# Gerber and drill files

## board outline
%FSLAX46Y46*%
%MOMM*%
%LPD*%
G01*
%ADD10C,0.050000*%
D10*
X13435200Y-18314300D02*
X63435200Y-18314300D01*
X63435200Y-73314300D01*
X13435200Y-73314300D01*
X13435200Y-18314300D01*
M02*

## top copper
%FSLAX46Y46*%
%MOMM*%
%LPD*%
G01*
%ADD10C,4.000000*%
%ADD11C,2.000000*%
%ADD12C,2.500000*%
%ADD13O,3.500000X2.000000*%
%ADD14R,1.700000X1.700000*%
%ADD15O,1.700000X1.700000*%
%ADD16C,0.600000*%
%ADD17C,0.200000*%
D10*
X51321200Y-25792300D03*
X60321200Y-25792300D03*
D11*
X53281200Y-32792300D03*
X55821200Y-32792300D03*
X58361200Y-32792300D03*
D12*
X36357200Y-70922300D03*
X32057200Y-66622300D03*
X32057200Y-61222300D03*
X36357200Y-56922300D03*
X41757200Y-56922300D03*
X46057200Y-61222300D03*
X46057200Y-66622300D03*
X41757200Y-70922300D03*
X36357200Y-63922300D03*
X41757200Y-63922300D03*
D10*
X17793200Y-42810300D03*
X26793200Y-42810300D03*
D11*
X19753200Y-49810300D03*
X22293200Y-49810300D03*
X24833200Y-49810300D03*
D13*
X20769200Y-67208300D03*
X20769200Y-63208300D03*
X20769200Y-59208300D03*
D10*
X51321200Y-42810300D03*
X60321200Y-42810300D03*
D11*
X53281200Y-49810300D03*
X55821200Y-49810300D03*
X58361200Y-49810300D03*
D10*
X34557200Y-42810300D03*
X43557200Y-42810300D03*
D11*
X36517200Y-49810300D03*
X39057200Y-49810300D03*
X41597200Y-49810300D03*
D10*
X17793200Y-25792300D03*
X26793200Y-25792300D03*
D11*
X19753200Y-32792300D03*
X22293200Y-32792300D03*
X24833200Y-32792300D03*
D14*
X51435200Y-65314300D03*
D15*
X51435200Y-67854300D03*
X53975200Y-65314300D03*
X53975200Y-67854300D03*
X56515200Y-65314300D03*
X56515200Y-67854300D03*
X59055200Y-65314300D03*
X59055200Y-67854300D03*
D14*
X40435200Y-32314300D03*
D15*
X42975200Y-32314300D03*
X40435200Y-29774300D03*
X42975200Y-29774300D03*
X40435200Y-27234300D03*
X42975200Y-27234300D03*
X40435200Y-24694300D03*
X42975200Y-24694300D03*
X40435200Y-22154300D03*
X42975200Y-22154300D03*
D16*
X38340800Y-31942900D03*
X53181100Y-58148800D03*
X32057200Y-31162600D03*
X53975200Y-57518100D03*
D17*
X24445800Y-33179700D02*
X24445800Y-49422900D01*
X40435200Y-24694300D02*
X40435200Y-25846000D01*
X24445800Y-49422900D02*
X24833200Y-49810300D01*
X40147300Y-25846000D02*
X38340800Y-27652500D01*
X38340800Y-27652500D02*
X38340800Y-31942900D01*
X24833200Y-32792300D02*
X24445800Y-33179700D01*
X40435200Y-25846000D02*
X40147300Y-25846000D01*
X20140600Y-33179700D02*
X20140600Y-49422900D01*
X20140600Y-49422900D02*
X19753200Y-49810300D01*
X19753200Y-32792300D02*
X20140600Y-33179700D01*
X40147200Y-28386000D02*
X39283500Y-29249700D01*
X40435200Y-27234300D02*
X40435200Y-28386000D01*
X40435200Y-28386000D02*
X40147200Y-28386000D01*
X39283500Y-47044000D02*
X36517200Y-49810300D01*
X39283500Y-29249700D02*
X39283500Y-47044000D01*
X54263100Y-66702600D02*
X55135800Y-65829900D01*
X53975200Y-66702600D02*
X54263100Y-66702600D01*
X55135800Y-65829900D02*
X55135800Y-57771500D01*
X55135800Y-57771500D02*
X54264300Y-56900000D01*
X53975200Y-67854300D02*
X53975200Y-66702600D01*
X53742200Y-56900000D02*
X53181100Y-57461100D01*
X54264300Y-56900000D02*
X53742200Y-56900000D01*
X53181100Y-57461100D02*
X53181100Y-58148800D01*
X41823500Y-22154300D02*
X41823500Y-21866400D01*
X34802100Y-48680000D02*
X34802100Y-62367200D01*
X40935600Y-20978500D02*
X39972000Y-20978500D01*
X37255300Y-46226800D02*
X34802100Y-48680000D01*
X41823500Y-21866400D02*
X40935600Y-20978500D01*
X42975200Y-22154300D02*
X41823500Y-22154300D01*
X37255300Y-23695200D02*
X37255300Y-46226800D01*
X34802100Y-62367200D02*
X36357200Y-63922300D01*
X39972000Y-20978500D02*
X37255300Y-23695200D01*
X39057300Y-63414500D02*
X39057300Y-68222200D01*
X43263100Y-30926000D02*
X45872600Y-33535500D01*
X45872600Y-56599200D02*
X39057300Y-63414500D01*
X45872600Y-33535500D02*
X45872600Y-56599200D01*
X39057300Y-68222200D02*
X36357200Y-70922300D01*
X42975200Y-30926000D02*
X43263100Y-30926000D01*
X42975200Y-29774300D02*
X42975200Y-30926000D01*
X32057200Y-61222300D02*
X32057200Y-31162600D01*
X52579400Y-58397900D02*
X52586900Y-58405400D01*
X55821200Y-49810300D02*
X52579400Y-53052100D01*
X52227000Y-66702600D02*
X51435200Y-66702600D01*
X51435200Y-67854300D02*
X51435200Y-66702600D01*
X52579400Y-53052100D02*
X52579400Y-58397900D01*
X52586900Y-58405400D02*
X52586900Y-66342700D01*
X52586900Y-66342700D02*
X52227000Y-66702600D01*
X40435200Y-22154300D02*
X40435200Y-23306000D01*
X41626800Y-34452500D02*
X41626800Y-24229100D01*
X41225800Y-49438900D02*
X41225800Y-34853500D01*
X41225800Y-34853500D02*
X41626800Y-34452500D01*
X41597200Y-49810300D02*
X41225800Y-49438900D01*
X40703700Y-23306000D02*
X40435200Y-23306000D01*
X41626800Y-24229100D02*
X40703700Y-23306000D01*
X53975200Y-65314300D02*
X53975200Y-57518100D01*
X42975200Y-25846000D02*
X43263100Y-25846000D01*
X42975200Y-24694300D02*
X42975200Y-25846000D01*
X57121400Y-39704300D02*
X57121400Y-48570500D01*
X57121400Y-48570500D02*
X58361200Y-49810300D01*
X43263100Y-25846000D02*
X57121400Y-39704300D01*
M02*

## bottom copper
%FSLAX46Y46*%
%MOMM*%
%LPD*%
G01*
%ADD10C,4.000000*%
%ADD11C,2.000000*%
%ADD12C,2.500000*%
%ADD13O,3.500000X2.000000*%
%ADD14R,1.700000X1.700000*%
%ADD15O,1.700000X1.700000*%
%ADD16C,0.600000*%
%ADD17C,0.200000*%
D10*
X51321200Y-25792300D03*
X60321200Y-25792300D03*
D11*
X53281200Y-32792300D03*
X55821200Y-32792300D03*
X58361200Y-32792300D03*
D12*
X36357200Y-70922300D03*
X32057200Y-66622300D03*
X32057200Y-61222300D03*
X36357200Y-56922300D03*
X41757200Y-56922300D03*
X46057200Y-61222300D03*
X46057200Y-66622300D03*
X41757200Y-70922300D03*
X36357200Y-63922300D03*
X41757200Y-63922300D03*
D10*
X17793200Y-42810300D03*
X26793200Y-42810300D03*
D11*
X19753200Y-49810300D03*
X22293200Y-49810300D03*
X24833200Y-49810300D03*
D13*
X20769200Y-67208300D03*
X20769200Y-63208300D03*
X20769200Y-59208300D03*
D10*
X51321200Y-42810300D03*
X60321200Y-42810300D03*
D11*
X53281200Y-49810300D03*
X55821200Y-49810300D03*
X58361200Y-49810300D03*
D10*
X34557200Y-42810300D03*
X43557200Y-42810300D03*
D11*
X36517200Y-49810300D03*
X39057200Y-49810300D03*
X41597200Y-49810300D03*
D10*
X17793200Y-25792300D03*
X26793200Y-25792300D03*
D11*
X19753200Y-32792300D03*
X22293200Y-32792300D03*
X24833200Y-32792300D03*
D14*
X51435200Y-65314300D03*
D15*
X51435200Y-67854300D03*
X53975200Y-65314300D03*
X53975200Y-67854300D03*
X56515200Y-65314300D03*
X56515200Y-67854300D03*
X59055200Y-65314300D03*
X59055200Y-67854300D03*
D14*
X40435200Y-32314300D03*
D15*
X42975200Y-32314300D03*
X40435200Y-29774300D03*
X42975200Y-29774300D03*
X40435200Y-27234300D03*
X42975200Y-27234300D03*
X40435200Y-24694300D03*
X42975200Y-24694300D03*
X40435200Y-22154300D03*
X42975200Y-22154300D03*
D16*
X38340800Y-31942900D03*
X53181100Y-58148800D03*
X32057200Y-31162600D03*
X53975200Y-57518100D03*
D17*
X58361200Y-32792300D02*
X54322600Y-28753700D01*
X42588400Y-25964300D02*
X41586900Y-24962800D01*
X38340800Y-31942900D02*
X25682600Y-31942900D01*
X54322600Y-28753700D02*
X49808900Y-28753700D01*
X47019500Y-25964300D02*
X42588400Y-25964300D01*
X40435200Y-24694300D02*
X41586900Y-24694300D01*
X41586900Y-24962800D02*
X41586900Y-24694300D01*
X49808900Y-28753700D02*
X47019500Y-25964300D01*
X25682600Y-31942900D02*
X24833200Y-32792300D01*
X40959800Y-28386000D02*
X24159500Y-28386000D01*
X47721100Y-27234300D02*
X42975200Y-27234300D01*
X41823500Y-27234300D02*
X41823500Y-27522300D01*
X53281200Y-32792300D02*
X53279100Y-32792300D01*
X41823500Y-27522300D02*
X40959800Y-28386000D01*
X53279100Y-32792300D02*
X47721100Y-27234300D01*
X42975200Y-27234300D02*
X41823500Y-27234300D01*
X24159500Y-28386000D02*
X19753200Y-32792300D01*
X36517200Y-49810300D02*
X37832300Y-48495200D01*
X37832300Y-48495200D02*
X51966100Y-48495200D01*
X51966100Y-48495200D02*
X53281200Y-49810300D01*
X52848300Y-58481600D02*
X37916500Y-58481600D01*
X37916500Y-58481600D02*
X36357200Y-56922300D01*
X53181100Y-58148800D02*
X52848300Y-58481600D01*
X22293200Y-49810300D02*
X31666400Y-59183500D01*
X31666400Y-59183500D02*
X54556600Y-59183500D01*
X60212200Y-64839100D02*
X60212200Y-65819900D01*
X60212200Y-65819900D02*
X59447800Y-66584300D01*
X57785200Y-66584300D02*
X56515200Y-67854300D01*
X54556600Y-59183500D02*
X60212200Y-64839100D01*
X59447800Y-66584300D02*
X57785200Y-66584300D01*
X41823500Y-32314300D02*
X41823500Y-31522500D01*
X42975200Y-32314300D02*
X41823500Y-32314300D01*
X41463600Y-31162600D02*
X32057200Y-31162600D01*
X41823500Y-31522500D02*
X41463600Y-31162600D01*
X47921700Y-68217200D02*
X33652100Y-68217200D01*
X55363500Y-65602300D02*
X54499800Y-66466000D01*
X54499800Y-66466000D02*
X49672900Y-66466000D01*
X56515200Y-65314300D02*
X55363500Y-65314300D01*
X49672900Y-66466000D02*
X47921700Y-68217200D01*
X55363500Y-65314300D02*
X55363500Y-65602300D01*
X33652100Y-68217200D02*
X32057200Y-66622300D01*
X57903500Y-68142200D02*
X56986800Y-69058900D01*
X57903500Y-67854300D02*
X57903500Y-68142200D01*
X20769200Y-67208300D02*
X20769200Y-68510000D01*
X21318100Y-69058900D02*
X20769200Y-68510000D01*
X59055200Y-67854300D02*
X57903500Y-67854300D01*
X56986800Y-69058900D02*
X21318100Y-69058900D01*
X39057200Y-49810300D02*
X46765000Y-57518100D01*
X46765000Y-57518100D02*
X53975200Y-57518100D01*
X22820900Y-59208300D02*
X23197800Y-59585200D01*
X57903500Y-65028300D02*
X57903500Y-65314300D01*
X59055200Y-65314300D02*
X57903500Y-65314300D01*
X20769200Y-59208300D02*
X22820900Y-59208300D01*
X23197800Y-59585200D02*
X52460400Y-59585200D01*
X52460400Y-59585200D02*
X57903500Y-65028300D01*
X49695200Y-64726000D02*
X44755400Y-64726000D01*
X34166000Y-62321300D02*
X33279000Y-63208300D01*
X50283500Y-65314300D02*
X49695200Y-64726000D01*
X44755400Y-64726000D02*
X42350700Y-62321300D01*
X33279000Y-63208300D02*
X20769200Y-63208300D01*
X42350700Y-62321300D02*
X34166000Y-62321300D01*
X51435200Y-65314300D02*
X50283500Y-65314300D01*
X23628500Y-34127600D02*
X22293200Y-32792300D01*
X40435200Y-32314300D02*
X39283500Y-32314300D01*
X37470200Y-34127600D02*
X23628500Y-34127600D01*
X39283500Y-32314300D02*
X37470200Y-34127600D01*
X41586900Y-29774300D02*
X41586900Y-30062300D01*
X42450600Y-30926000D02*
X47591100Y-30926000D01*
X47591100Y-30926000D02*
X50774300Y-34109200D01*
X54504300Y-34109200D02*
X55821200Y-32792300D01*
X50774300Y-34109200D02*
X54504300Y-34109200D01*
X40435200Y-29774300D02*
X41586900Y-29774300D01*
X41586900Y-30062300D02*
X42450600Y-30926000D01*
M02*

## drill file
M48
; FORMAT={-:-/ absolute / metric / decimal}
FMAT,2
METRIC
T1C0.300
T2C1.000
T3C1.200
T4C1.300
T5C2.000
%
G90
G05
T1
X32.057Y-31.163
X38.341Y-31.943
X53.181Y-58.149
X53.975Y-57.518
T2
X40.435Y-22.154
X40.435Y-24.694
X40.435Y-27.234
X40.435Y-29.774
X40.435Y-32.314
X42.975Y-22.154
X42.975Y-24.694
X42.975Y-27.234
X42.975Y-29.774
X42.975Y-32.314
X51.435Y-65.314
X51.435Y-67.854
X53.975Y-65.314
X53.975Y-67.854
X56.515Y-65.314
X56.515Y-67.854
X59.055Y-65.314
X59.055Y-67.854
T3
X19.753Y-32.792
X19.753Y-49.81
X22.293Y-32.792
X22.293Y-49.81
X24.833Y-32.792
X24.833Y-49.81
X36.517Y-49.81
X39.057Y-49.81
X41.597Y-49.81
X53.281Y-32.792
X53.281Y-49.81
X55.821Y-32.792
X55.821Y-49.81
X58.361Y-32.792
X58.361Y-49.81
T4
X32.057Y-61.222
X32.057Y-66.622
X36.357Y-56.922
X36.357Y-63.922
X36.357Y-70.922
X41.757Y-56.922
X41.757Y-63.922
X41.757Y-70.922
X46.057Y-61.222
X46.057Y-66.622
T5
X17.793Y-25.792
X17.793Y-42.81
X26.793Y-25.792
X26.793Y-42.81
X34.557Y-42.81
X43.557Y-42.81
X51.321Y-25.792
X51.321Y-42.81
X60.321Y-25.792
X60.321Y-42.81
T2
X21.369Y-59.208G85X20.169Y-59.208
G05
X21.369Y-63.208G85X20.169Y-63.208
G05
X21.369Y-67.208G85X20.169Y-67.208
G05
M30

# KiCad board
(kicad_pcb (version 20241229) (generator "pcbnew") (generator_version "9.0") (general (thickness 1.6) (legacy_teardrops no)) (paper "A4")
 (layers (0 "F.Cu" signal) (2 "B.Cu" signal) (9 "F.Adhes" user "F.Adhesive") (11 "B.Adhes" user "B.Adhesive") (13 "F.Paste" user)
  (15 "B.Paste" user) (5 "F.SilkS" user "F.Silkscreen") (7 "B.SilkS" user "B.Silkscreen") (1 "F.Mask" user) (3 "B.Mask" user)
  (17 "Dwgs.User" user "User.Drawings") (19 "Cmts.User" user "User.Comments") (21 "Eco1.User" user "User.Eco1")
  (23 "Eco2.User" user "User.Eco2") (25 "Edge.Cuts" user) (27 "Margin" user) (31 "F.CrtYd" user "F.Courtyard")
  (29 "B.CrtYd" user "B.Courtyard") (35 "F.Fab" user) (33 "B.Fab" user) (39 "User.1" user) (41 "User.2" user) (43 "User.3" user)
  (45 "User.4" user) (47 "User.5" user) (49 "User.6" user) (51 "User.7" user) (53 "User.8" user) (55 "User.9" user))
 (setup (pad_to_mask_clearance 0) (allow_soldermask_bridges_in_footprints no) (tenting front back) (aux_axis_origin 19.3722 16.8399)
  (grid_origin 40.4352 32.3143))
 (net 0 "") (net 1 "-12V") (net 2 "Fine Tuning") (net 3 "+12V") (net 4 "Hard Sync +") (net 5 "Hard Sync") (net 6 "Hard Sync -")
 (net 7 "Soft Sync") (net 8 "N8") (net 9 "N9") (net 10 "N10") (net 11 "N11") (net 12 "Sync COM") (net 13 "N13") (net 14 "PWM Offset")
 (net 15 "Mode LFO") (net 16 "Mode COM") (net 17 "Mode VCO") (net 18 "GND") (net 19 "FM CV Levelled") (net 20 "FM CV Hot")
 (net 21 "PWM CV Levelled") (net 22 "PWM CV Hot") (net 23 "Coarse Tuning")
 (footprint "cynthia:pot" (layer "F.Cu") (at 55.8212 25.7923)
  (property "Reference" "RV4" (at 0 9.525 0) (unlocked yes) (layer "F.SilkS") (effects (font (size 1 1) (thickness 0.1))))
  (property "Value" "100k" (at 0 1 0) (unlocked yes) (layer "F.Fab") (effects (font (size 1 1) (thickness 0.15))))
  (pad "" np_thru_hole circle (at -4.5 0) (size 4 4) (drill 2) (layers "*.Cu" "*.Mask"))
  (pad "" np_thru_hole circle (at 4.5 0) (size 4 4) (drill 2) (layers "*.Cu" "*.Mask"))
  (pad "1" thru_hole circle (at -2.54 7) (size 2 2) (drill 1.2) (layers "*.Cu" "*.Mask") (remove_unused_layers no) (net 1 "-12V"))
  (pad "2" thru_hole circle (at 0 7) (size 2 2) (drill 1.2) (layers "*.Cu" "*.Mask") (remove_unused_layers no) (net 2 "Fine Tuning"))
  (pad "3" thru_hole circle (at 2.54 7) (size 2 2) (drill 1.2) (layers "*.Cu" "*.Mask") (remove_unused_layers no) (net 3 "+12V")))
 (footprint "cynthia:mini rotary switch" (layer "F.Cu") (at 39.0572 63.9223)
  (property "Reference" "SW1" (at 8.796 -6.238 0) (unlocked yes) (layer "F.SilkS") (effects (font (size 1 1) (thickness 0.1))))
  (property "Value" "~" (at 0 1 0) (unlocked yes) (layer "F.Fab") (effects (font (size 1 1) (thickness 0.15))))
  (pad "1" thru_hole circle (at -2.7 7 135) (size 2.5 2.5) (drill 1.3) (layers "*.Cu" "*.Mask") (remove_unused_layers no)
   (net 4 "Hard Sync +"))
  (pad "2" thru_hole circle (at -7 2.7 135) (size 2.5 2.5) (drill 1.3) (layers "*.Cu" "*.Mask") (remove_unused_layers no)
   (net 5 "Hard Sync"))
  (pad "3" thru_hole circle (at -7 -2.7 135) (size 2.5 2.5) (drill 1.3) (layers "*.Cu" "*.Mask") (remove_unused_layers no)
   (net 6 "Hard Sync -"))
  (pad "4" thru_hole circle (at -2.7 -7 135) (size 2.5 2.5) (drill 1.3) (layers "*.Cu" "*.Mask") (remove_unused_layers no)
   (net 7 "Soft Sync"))
  (pad "5" thru_hole circle (at 2.7 -7 135) (size 2.5 2.5) (drill 1.3) (layers "*.Cu" "*.Mask") (remove_unused_layers no) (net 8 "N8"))
  (pad "6" thru_hole circle (at 7 -2.7 135) (size 2.5 2.5) (drill 1.3) (layers "*.Cu" "*.Mask") (remove_unused_layers no) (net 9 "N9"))
  (pad "7" thru_hole circle (at 7 2.7 135) (size 2.5 2.5) (drill 1.3) (layers "*.Cu" "*.Mask") (remove_unused_layers no) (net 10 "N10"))
  (pad "8" thru_hole circle (at 2.7 7 135) (size 2.5 2.5) (drill 1.3) (layers "*.Cu" "*.Mask") (remove_unused_layers no) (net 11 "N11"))
  (pad "9" thru_hole circle (at -2.7 0 135) (size 2.5 2.5) (drill 1.3) (layers "*.Cu" "*.Mask") (remove_unused_layers no)
   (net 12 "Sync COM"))
  (pad "10" thru_hole circle (at 2.7 0 135) (size 2.5 2.5) (drill 1.3) (layers "*.Cu" "*.Mask") (remove_unused_layers no) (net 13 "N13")))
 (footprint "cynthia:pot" (layer "F.Cu") (at 22.2932 42.8103)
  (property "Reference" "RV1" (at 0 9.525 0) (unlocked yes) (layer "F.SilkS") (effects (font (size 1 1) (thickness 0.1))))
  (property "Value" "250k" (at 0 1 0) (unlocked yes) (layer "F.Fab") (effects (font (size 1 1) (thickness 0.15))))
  (pad "" np_thru_hole circle (at -4.5 0) (size 4 4) (drill 2) (layers "*.Cu" "*.Mask"))
  (pad "" np_thru_hole circle (at 4.5 0) (size 4 4) (drill 2) (layers "*.Cu" "*.Mask"))
  (pad "1" thru_hole circle (at -2.54 7) (size 2 2) (drill 1.2) (layers "*.Cu" "*.Mask") (remove_unused_layers no) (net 1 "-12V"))
  (pad "2" thru_hole circle (at 0 7) (size 2 2) (drill 1.2) (layers "*.Cu" "*.Mask") (remove_unused_layers no) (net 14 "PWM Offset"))
  (pad "3" thru_hole circle (at 2.54 7) (size 2 2) (drill 1.2) (layers "*.Cu" "*.Mask") (remove_unused_layers no) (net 3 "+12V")))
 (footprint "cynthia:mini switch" (layer "F.Cu") (at 20.7692 63.2083 90)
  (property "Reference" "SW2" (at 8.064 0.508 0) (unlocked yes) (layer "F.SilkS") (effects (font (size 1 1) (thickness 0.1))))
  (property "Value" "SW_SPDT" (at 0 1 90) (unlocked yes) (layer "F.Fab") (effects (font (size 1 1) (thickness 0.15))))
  (pad "1" thru_hole oval (at -4 0 180) (size 3.5 2) (drill oval 2.2 1) (layers "*.Cu" "*.Mask") (remove_unused_layers no)
   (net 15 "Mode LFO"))
  (pad "2" thru_hole oval (at 0 0 180) (size 3.5 2) (drill oval 2.2 1) (layers "*.Cu" "*.Mask") (remove_unused_layers no)
   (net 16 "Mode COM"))
  (pad "3" thru_hole oval (at 4 0 180) (size 3.5 2) (drill oval 2.2 1) (layers "*.Cu" "*.Mask") (remove_unused_layers no)
   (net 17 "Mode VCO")))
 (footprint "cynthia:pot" (layer "F.Cu") (at 55.8212 42.8103)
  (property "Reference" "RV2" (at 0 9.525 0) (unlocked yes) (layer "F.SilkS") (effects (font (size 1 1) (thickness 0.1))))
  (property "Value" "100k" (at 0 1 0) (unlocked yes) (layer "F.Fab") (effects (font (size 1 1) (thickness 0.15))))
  (pad "" np_thru_hole circle (at -4.5 0) (size 4 4) (drill 2) (layers "*.Cu" "*.Mask"))
  (pad "" np_thru_hole circle (at 4.5 0) (size 4 4) (drill 2) (layers "*.Cu" "*.Mask"))
  (pad "1" thru_hole circle (at -2.54 7) (size 2 2) (drill 1.2) (layers "*.Cu" "*.Mask") (remove_unused_layers no) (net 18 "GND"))
  (pad "2" thru_hole circle (at 0 7) (size 2 2) (drill 1.2) (layers "*.Cu" "*.Mask") (remove_unused_layers no) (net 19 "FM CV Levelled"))
  (pad "3" thru_hole circle (at 2.54 7) (size 2 2) (drill 1.2) (layers "*.Cu" "*.Mask") (remove_unused_layers no) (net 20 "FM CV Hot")))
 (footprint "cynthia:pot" (layer "F.Cu") (at 39.0572 42.8103)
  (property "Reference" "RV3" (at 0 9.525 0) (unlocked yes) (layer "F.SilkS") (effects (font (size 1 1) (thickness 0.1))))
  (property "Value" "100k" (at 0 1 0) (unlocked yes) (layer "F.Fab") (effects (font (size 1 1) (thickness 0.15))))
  (pad "" np_thru_hole circle (at -4.5 0) (size 4 4) (drill 2) (layers "*.Cu" "*.Mask"))
  (pad "" np_thru_hole circle (at 4.5 0) (size 4 4) (drill 2) (layers "*.Cu" "*.Mask"))
  (pad "1" thru_hole circle (at -2.54 7) (size 2 2) (drill 1.2) (layers "*.Cu" "*.Mask") (remove_unused_layers no) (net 18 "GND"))
  (pad "2" thru_hole circle (at 0 7) (size 2 2) (drill 1.2) (layers "*.Cu" "*.Mask") (remove_unused_layers no) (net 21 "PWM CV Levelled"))
  (pad "3" thru_hole circle (at 2.54 7) (size 2 2) (drill 1.2) (layers "*.Cu" "*.Mask") (remove_unused_layers no) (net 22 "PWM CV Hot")))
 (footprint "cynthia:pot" (layer "F.Cu") (at 22.2932 25.7923)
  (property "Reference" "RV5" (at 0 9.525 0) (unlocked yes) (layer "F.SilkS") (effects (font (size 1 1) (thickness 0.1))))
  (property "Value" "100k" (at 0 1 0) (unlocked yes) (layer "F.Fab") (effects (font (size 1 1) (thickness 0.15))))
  (pad "" np_thru_hole circle (at -4.5 0) (size 4 4) (drill 2) (layers "*.Cu" "*.Mask"))
  (pad "" np_thru_hole circle (at 4.5 0) (size 4 4) (drill 2) (layers "*.Cu" "*.Mask"))
  (pad "1" thru_hole circle (at -2.54 7) (size 2 2) (drill 1.2) (layers "*.Cu" "*.Mask") (remove_unused_layers no) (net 1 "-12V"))
  (pad "2" thru_hole circle (at 0 7) (size 2 2) (drill 1.2) (layers "*.Cu" "*.Mask") (remove_unused_layers no) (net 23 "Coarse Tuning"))
  (pad "3" thru_hole circle (at 2.54 7) (size 2 2) (drill 1.2) (layers "*.Cu" "*.Mask") (remove_unused_layers no) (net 3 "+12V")))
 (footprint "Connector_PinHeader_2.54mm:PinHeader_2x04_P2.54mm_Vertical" (layer "B.Cu") (at 51.4352 65.3143 -90)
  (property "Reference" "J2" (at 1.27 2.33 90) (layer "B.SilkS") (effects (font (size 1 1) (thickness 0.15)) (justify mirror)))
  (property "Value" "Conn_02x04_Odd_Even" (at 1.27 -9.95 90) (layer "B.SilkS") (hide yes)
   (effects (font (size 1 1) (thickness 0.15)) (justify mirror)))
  (pad "1" thru_hole rect (at 0 0 270) (size 1.7 1.7) (drill 1) (layers "*.Cu" "*.Mask") (remove_unused_layers no) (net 16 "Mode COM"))
  (pad "2" thru_hole oval (at 2.54 0 270) (size 1.7 1.7) (drill 1) (layers "*.Cu" "*.Mask") (remove_unused_layers no)
   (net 19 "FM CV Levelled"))
  (pad "3" thru_hole oval (at 0 -2.54 270) (size 1.7 1.7) (drill 1) (layers "*.Cu" "*.Mask") (remove_unused_layers no)
   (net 21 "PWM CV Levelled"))
  (pad "4" thru_hole oval (at 2.54 -2.54 270) (size 1.7 1.7) (drill 1) (layers "*.Cu" "*.Mask") (remove_unused_layers no)
   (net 7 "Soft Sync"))
  (pad "5" thru_hole oval (at 0 -5.08 270) (size 1.7 1.7) (drill 1) (layers "*.Cu" "*.Mask") (remove_unused_layers no) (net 5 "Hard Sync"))
  (pad "6" thru_hole oval (at 2.54 -5.08 270) (size 1.7 1.7) (drill 1) (layers "*.Cu" "*.Mask") (remove_unused_layers no)
   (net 14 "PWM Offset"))
  (pad "7" thru_hole oval (at 0 -7.62 270) (size 1.7 1.7) (drill 1) (layers "*.Cu" "*.Mask") (remove_unused_layers no) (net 17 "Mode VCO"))
  (pad "8" thru_hole oval (at 2.54 -7.62 270) (size 1.7 1.7) (drill 1) (layers "*.Cu" "*.Mask") (remove_unused_layers no)
   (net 15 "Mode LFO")))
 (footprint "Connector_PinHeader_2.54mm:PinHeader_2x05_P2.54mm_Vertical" (layer "B.Cu") (at 40.4352 32.3143)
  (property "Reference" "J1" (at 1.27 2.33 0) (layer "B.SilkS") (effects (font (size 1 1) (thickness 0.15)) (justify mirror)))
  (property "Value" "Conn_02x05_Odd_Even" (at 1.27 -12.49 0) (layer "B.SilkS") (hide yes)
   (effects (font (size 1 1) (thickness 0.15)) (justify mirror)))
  (pad "1" thru_hole rect (at 0 0) (size 1.7 1.7) (drill 1) (layers "*.Cu" "*.Mask") (remove_unused_layers no) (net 23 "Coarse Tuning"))
  (pad "2" thru_hole oval (at 2.54 0) (size 1.7 1.7) (drill 1) (layers "*.Cu" "*.Mask") (remove_unused_layers no) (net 6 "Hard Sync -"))
  (pad "3" thru_hole oval (at 0 -2.54) (size 1.7 1.7) (drill 1) (layers "*.Cu" "*.Mask") (remove_unused_layers no) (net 2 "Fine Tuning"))
  (pad "4" thru_hole oval (at 2.54 -2.54) (size 1.7 1.7) (drill 1) (layers "*.Cu" "*.Mask") (remove_unused_layers no) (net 4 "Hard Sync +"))
  (pad "5" thru_hole oval (at 0 -5.08) (size 1.7 1.7) (drill 1) (layers "*.Cu" "*.Mask") (remove_unused_layers no) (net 18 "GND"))
  (pad "6" thru_hole oval (at 2.54 -5.08) (size 1.7 1.7) (drill 1) (layers "*.Cu" "*.Mask") (remove_unused_layers no) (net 1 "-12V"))
  (pad "7" thru_hole oval (at 0 -7.62) (size 1.7 1.7) (drill 1) (layers "*.Cu" "*.Mask") (remove_unused_layers no) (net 3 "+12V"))
  (pad "8" thru_hole oval (at 2.54 -7.62) (size 1.7 1.7) (drill 1) (layers "*.Cu" "*.Mask") (remove_unused_layers no) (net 20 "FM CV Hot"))
  (pad "9" thru_hole oval (at 0 -10.16) (size 1.7 1.7) (drill 1) (layers "*.Cu" "*.Mask") (remove_unused_layers no) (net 22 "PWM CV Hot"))
  (pad "10" thru_hole oval (at 2.54 -10.16) (size 1.7 1.7) (drill 1) (layers "*.Cu" "*.Mask") (remove_unused_layers no) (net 12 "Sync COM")))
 (gr_rect (start 13.4352 18.3143) (end 63.4352 73.3143) (stroke (width 0.05) (type solid)) (fill no) (layer "Edge.Cuts"))
 (segment (start 24.4458 33.1797) (end 24.4458 49.4229) (width 0.2) (layer "F.Cu") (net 3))
 (segment (start 40.4352 24.6943) (end 40.4352 25.846) (width 0.2) (layer "F.Cu") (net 3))
 (segment (start 24.4458 49.4229) (end 24.8332 49.8103) (width 0.2) (layer "F.Cu") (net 3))
 (segment (start 40.1473 25.846) (end 38.3408 27.6525) (width 0.2) (layer "F.Cu") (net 3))
 (segment (start 38.3408 27.6525) (end 38.3408 31.9429) (width 0.2) (layer "F.Cu") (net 3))
 (segment (start 24.8332 32.7923) (end 24.4458 33.1797) (width 0.2) (layer "F.Cu") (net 3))
 (segment (start 40.4352 25.846) (end 40.1473 25.846) (width 0.2) (layer "F.Cu") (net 3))
 (via (at 38.3408 31.9429) (size 0.6) (drill 0.3) (layers "F.Cu" "B.Cu") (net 3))
 (segment (start 58.3612 32.7923) (end 54.3226 28.7537) (width 0.2) (layer "B.Cu") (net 3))
 (segment (start 42.5884 25.9643) (end 41.5869 24.9628) (width 0.2) (layer "B.Cu") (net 3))
 (segment (start 38.3408 31.9429) (end 25.6826 31.9429) (width 0.2) (layer "B.Cu") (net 3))
 (segment (start 54.3226 28.7537) (end 49.8089 28.7537) (width 0.2) (layer "B.Cu") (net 3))
 (segment (start 47.0195 25.9643) (end 42.5884 25.9643) (width 0.2) (layer "B.Cu") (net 3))
 (segment (start 40.4352 24.6943) (end 41.5869 24.6943) (width 0.2) (layer "B.Cu") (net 3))
 (segment (start 41.5869 24.9628) (end 41.5869 24.6943) (width 0.2) (layer "B.Cu") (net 3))
 (segment (start 49.8089 28.7537) (end 47.0195 25.9643) (width 0.2) (layer "B.Cu") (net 3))
 (segment (start 25.6826 31.9429) (end 24.8332 32.7923) (width 0.2) (layer "B.Cu") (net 3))
 (segment (start 20.1406 33.1797) (end 20.1406 49.4229) (width 0.2) (layer "F.Cu") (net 1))
 (segment (start 20.1406 49.4229) (end 19.7532 49.8103) (width 0.2) (layer "F.Cu") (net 1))
 (segment (start 19.7532 32.7923) (end 20.1406 33.1797) (width 0.2) (layer "F.Cu") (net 1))
 (segment (start 40.9598 28.386) (end 24.1595 28.386) (width 0.2) (layer "B.Cu") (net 1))
 (segment (start 47.7211 27.2343) (end 42.9752 27.2343) (width 0.2) (layer "B.Cu") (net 1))
 (segment (start 41.8235 27.2343) (end 41.8235 27.5223) (width 0.2) (layer "B.Cu") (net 1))
 (segment (start 53.2812 32.7923) (end 53.2791 32.7923) (width 0.2) (layer "B.Cu") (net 1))
 (segment (start 41.8235 27.5223) (end 40.9598 28.386) (width 0.2) (layer "B.Cu") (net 1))
 (segment (start 53.2791 32.7923) (end 47.7211 27.2343) (width 0.2) (layer "B.Cu") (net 1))
 (segment (start 42.9752 27.2343) (end 41.8235 27.2343) (width 0.2) (layer "B.Cu") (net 1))
 (segment (start 24.1595 28.386) (end 19.7532 32.7923) (width 0.2) (layer "B.Cu") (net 1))
 (segment (start 40.1472 28.386) (end 39.2835 29.2497) (width 0.2) (layer "F.Cu") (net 18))
 (segment (start 40.4352 27.2343) (end 40.4352 28.386) (width 0.2) (layer "F.Cu") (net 18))
 (segment (start 40.4352 28.386) (end 40.1472 28.386) (width 0.2) (layer "F.Cu") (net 18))
 (segment (start 39.2835 47.044) (end 36.5172 49.8103) (width 0.2) (layer "F.Cu") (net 18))
 (segment (start 39.2835 29.2497) (end 39.2835 47.044) (width 0.2) (layer "F.Cu") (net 18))
 (segment (start 36.5172 49.8103) (end 37.8323 48.4952) (width 0.2) (layer "B.Cu") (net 18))
 (segment (start 37.8323 48.4952) (end 51.9661 48.4952) (width 0.2) (layer "B.Cu") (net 18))
 (segment (start 51.9661 48.4952) (end 53.2812 49.8103) (width 0.2) (layer "B.Cu") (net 18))
 (segment (start 54.2631 66.7026) (end 55.1358 65.8299) (width 0.2) (layer "F.Cu") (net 7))
 (segment (start 53.9752 66.7026) (end 54.2631 66.7026) (width 0.2) (layer "F.Cu") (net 7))
 (segment (start 55.1358 65.8299) (end 55.1358 57.7715) (width 0.2) (layer "F.Cu") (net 7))
 (segment (start 55.1358 57.7715) (end 54.2643 56.9) (width 0.2) (layer "F.Cu") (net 7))
 (segment (start 53.9752 67.8543) (end 53.9752 66.7026) (width 0.2) (layer "F.Cu") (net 7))
 (segment (start 53.7422 56.9) (end 53.1811 57.4611) (width 0.2) (layer "F.Cu") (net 7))
 (segment (start 54.2643 56.9) (end 53.7422 56.9) (width 0.2) (layer "F.Cu") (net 7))
 (segment (start 53.1811 57.4611) (end 53.1811 58.1488) (width 0.2) (layer "F.Cu") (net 7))
 (via (at 53.1811 58.1488) (size 0.6) (drill 0.3) (layers "F.Cu" "B.Cu") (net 7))
 (segment (start 52.8483 58.4816) (end 37.9165 58.4816) (width 0.2) (layer "B.Cu") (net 7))
 (segment (start 37.9165 58.4816) (end 36.3572 56.9223) (width 0.2) (layer "B.Cu") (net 7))
 (segment (start 53.1811 58.1488) (end 52.8483 58.4816) (width 0.2) (layer "B.Cu") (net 7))
 (segment (start 41.8235 22.1543) (end 41.8235 21.8664) (width 0.2) (layer "F.Cu") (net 12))
 (segment (start 34.8021 48.68) (end 34.8021 62.3672) (width 0.2) (layer "F.Cu") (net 12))
 (segment (start 40.9356 20.9785) (end 39.972 20.9785) (width 0.2) (layer "F.Cu") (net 12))
 (segment (start 37.2553 46.2268) (end 34.8021 48.68) (width 0.2) (layer "F.Cu") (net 12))
 (segment (start 41.8235 21.8664) (end 40.9356 20.9785) (width 0.2) (layer "F.Cu") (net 12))
 (segment (start 42.9752 22.1543) (end 41.8235 22.1543) (width 0.2) (layer "F.Cu") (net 12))
 (segment (start 37.2553 23.6952) (end 37.2553 46.2268) (width 0.2) (layer "F.Cu") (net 12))
 (segment (start 34.8021 62.3672) (end 36.3572 63.9223) (width 0.2) (layer "F.Cu") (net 12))
 (segment (start 39.972 20.9785) (end 37.2553 23.6952) (width 0.2) (layer "F.Cu") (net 12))
 (segment (start 22.2932 49.8103) (end 31.6664 59.1835) (width 0.2) (layer "B.Cu") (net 14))
 (segment (start 31.6664 59.1835) (end 54.5566 59.1835) (width 0.2) (layer "B.Cu") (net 14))
 (segment (start 60.2122 64.8391) (end 60.2122 65.8199) (width 0.2) (layer "B.Cu") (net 14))
 (segment (start 60.2122 65.8199) (end 59.4478 66.5843) (width 0.2) (layer "B.Cu") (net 14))
 (segment (start 57.7852 66.5843) (end 56.5152 67.8543) (width 0.2) (layer "B.Cu") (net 14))
 (segment (start 54.5566 59.1835) (end 60.2122 64.8391) (width 0.2) (layer "B.Cu") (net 14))
 (segment (start 59.4478 66.5843) (end 57.7852 66.5843) (width 0.2) (layer "B.Cu") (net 14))
 (segment (start 39.0573 63.4145) (end 39.0573 68.2222) (width 0.2) (layer "F.Cu") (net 4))
 (segment (start 43.2631 30.926) (end 45.8726 33.5355) (width 0.2) (layer "F.Cu") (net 4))
 (segment (start 45.8726 56.5992) (end 39.0573 63.4145) (width 0.2) (layer "F.Cu") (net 4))
 (segment (start 45.8726 33.5355) (end 45.8726 56.5992) (width 0.2) (layer "F.Cu") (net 4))
 (segment (start 39.0573 68.2222) (end 36.3572 70.9223) (width 0.2) (layer "F.Cu") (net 4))
 (segment (start 42.9752 30.926) (end 43.2631 30.926) (width 0.2) (layer "F.Cu") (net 4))
 (segment (start 42.9752 29.7743) (end 42.9752 30.926) (width 0.2) (layer "F.Cu") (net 4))
 (segment (start 32.0572 61.2223) (end 32.0572 31.1626) (width 0.2) (layer "F.Cu") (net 6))
 (via (at 32.0572 31.1626) (size 0.6) (drill 0.3) (layers "F.Cu" "B.Cu") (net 6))
 (segment (start 41.8235 32.3143) (end 41.8235 31.5225) (width 0.2) (layer "B.Cu") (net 6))
 (segment (start 42.9752 32.3143) (end 41.8235 32.3143) (width 0.2) (layer "B.Cu") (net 6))
 (segment (start 41.4636 31.1626) (end 32.0572 31.1626) (width 0.2) (layer "B.Cu") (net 6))
 (segment (start 41.8235 31.5225) (end 41.4636 31.1626) (width 0.2) (layer "B.Cu") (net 6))
 (segment (start 47.9217 68.2172) (end 33.6521 68.2172) (width 0.2) (layer "B.Cu") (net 5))
 (segment (start 55.3635 65.6023) (end 54.4998 66.466) (width 0.2) (layer "B.Cu") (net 5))
 (segment (start 54.4998 66.466) (end 49.6729 66.466) (width 0.2) (layer "B.Cu") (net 5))
 (segment (start 56.5152 65.3143) (end 55.3635 65.3143) (width 0.2) (layer "B.Cu") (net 5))
 (segment (start 49.6729 66.466) (end 47.9217 68.2172) (width 0.2) (layer "B.Cu") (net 5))
 (segment (start 55.3635 65.3143) (end 55.3635 65.6023) (width 0.2) (layer "B.Cu") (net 5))
 (segment (start 33.6521 68.2172) (end 32.0572 66.6223) (width 0.2) (layer "B.Cu") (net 5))
 (segment (start 52.5794 58.3979) (end 52.5869 58.4054) (width 0.2) (layer "F.Cu") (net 19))
 (segment (start 55.8212 49.8103) (end 52.5794 53.0521) (width 0.2) (layer "F.Cu") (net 19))
 (segment (start 52.227 66.7026) (end 51.4352 66.7026) (width 0.2) (layer "F.Cu") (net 19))
 (segment (start 51.4352 67.8543) (end 51.4352 66.7026) (width 0.2) (layer "F.Cu") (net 19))
 (segment (start 52.5794 53.0521) (end 52.5794 58.3979) (width 0.2) (layer "F.Cu") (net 19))
 (segment (start 52.5869 58.4054) (end 52.5869 66.3427) (width 0.2) (layer "F.Cu") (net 19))
 (segment (start 52.5869 66.3427) (end 52.227 66.7026) (width 0.2) (layer "F.Cu") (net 19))
 (segment (start 57.9035 68.1422) (end 56.9868 69.0589) (width 0.2) (layer "B.Cu") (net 15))
 (segment (start 57.9035 67.8543) (end 57.9035 68.1422) (width 0.2) (layer "B.Cu") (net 15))
 (segment (start 20.7692 67.2083) (end 20.7692 68.51) (width 0.2) (layer "B.Cu") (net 15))
 (segment (start 21.3181 69.0589) (end 20.7692 68.51) (width 0.2) (layer "B.Cu") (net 15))
 (segment (start 59.0552 67.8543) (end 57.9035 67.8543) (width 0.2) (layer "B.Cu") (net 15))
 (segment (start 56.9868 69.0589) (end 21.3181 69.0589) (width 0.2) (layer "B.Cu") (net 15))
 (segment (start 40.4352 22.1543) (end 40.4352 23.306) (width 0.2) (layer "F.Cu") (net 22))
 (segment (start 41.6268 34.4525) (end 41.6268 24.2291) (width 0.2) (layer "F.Cu") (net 22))
 (segment (start 41.2258 49.4389) (end 41.2258 34.8535) (width 0.2) (layer "F.Cu") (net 22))
 (segment (start 41.2258 34.8535) (end 41.6268 34.4525) (width 0.2) (layer "F.Cu") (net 22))
 (segment (start 41.5972 49.8103) (end 41.2258 49.4389) (width 0.2) (layer "F.Cu") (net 22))
 (segment (start 40.7037 23.306) (end 40.4352 23.306) (width 0.2) (layer "F.Cu") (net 22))
 (segment (start 41.6268 24.2291) (end 40.7037 23.306) (width 0.2) (layer "F.Cu") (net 22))
 (segment (start 53.9752 65.3143) (end 53.9752 57.5181) (width 0.2) (layer "F.Cu") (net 21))
 (via (at 53.9752 57.5181) (size 0.6) (drill 0.3) (layers "F.Cu" "B.Cu") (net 21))
 (segment (start 39.0572 49.8103) (end 46.765 57.5181) (width 0.2) (layer "B.Cu") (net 21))
 (segment (start 46.765 57.5181) (end 53.9752 57.5181) (width 0.2) (layer "B.Cu") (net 21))
 (segment (start 22.8209 59.2083) (end 23.1978 59.5852) (width 0.2) (layer "B.Cu") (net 17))
 (segment (start 57.9035 65.0283) (end 57.9035 65.3143) (width 0.2) (layer "B.Cu") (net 17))
 (segment (start 59.0552 65.3143) (end 57.9035 65.3143) (width 0.2) (layer "B.Cu") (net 17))
 (segment (start 20.7692 59.2083) (end 22.8209 59.2083) (width 0.2) (layer "B.Cu") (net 17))
 (segment (start 23.1978 59.5852) (end 52.4604 59.5852) (width 0.2) (layer "B.Cu") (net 17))
 (segment (start 52.4604 59.5852) (end 57.9035 65.0283) (width 0.2) (layer "B.Cu") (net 17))
 (segment (start 42.9752 25.846) (end 43.2631 25.846) (width 0.2) (layer "F.Cu") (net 20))
 (segment (start 42.9752 24.6943) (end 42.9752 25.846) (width 0.2) (layer "F.Cu") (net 20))
 (segment (start 57.1214 39.7043) (end 57.1214 48.5705) (width 0.2) (layer "F.Cu") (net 20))
 (segment (start 57.1214 48.5705) (end 58.3612 49.8103) (width 0.2) (layer "F.Cu") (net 20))
 (segment (start 43.2631 25.846) (end 57.1214 39.7043) (width 0.2) (layer "F.Cu") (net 20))
 (segment (start 49.6952 64.726) (end 44.7554 64.726) (width 0.2) (layer "B.Cu") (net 16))
 (segment (start 34.166 62.3213) (end 33.279 63.2083) (width 0.2) (layer "B.Cu") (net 16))
 (segment (start 50.2835 65.3143) (end 49.6952 64.726) (width 0.2) (layer "B.Cu") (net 16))
 (segment (start 44.7554 64.726) (end 42.3507 62.3213) (width 0.2) (layer "B.Cu") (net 16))
 (segment (start 33.279 63.2083) (end 20.7692 63.2083) (width 0.2) (layer "B.Cu") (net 16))
 (segment (start 42.3507 62.3213) (end 34.166 62.3213) (width 0.2) (layer "B.Cu") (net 16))
 (segment (start 51.4352 65.3143) (end 50.2835 65.3143) (width 0.2) (layer "B.Cu") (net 16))
 (segment (start 23.6285 34.1276) (end 22.2932 32.7923) (width 0.2) (layer "B.Cu") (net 23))
 (segment (start 40.4352 32.3143) (end 39.2835 32.3143) (width 0.2) (layer "B.Cu") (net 23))
 (segment (start 37.4702 34.1276) (end 23.6285 34.1276) (width 0.2) (layer "B.Cu") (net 23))
 (segment (start 39.2835 32.3143) (end 37.4702 34.1276) (width 0.2) (layer "B.Cu") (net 23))
 (segment (start 41.5869 29.7743) (end 41.5869 30.0623) (width 0.2) (layer "B.Cu") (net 2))
 (segment (start 42.4506 30.926) (end 47.5911 30.926) (width 0.2) (layer "B.Cu") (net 2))
 (segment (start 47.5911 30.926) (end 50.7743 34.1092) (width 0.2) (layer "B.Cu") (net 2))
 (segment (start 54.5043 34.1092) (end 55.8212 32.7923) (width 0.2) (layer "B.Cu") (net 2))
 (segment (start 50.7743 34.1092) (end 54.5043 34.1092) (width 0.2) (layer "B.Cu") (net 2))
 (segment (start 40.4352 29.7743) (end 41.5869 29.7743) (width 0.2) (layer "B.Cu") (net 2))
 (segment (start 41.5869 30.0623) (end 42.4506 30.926) (width 0.2) (layer "B.Cu") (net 2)))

